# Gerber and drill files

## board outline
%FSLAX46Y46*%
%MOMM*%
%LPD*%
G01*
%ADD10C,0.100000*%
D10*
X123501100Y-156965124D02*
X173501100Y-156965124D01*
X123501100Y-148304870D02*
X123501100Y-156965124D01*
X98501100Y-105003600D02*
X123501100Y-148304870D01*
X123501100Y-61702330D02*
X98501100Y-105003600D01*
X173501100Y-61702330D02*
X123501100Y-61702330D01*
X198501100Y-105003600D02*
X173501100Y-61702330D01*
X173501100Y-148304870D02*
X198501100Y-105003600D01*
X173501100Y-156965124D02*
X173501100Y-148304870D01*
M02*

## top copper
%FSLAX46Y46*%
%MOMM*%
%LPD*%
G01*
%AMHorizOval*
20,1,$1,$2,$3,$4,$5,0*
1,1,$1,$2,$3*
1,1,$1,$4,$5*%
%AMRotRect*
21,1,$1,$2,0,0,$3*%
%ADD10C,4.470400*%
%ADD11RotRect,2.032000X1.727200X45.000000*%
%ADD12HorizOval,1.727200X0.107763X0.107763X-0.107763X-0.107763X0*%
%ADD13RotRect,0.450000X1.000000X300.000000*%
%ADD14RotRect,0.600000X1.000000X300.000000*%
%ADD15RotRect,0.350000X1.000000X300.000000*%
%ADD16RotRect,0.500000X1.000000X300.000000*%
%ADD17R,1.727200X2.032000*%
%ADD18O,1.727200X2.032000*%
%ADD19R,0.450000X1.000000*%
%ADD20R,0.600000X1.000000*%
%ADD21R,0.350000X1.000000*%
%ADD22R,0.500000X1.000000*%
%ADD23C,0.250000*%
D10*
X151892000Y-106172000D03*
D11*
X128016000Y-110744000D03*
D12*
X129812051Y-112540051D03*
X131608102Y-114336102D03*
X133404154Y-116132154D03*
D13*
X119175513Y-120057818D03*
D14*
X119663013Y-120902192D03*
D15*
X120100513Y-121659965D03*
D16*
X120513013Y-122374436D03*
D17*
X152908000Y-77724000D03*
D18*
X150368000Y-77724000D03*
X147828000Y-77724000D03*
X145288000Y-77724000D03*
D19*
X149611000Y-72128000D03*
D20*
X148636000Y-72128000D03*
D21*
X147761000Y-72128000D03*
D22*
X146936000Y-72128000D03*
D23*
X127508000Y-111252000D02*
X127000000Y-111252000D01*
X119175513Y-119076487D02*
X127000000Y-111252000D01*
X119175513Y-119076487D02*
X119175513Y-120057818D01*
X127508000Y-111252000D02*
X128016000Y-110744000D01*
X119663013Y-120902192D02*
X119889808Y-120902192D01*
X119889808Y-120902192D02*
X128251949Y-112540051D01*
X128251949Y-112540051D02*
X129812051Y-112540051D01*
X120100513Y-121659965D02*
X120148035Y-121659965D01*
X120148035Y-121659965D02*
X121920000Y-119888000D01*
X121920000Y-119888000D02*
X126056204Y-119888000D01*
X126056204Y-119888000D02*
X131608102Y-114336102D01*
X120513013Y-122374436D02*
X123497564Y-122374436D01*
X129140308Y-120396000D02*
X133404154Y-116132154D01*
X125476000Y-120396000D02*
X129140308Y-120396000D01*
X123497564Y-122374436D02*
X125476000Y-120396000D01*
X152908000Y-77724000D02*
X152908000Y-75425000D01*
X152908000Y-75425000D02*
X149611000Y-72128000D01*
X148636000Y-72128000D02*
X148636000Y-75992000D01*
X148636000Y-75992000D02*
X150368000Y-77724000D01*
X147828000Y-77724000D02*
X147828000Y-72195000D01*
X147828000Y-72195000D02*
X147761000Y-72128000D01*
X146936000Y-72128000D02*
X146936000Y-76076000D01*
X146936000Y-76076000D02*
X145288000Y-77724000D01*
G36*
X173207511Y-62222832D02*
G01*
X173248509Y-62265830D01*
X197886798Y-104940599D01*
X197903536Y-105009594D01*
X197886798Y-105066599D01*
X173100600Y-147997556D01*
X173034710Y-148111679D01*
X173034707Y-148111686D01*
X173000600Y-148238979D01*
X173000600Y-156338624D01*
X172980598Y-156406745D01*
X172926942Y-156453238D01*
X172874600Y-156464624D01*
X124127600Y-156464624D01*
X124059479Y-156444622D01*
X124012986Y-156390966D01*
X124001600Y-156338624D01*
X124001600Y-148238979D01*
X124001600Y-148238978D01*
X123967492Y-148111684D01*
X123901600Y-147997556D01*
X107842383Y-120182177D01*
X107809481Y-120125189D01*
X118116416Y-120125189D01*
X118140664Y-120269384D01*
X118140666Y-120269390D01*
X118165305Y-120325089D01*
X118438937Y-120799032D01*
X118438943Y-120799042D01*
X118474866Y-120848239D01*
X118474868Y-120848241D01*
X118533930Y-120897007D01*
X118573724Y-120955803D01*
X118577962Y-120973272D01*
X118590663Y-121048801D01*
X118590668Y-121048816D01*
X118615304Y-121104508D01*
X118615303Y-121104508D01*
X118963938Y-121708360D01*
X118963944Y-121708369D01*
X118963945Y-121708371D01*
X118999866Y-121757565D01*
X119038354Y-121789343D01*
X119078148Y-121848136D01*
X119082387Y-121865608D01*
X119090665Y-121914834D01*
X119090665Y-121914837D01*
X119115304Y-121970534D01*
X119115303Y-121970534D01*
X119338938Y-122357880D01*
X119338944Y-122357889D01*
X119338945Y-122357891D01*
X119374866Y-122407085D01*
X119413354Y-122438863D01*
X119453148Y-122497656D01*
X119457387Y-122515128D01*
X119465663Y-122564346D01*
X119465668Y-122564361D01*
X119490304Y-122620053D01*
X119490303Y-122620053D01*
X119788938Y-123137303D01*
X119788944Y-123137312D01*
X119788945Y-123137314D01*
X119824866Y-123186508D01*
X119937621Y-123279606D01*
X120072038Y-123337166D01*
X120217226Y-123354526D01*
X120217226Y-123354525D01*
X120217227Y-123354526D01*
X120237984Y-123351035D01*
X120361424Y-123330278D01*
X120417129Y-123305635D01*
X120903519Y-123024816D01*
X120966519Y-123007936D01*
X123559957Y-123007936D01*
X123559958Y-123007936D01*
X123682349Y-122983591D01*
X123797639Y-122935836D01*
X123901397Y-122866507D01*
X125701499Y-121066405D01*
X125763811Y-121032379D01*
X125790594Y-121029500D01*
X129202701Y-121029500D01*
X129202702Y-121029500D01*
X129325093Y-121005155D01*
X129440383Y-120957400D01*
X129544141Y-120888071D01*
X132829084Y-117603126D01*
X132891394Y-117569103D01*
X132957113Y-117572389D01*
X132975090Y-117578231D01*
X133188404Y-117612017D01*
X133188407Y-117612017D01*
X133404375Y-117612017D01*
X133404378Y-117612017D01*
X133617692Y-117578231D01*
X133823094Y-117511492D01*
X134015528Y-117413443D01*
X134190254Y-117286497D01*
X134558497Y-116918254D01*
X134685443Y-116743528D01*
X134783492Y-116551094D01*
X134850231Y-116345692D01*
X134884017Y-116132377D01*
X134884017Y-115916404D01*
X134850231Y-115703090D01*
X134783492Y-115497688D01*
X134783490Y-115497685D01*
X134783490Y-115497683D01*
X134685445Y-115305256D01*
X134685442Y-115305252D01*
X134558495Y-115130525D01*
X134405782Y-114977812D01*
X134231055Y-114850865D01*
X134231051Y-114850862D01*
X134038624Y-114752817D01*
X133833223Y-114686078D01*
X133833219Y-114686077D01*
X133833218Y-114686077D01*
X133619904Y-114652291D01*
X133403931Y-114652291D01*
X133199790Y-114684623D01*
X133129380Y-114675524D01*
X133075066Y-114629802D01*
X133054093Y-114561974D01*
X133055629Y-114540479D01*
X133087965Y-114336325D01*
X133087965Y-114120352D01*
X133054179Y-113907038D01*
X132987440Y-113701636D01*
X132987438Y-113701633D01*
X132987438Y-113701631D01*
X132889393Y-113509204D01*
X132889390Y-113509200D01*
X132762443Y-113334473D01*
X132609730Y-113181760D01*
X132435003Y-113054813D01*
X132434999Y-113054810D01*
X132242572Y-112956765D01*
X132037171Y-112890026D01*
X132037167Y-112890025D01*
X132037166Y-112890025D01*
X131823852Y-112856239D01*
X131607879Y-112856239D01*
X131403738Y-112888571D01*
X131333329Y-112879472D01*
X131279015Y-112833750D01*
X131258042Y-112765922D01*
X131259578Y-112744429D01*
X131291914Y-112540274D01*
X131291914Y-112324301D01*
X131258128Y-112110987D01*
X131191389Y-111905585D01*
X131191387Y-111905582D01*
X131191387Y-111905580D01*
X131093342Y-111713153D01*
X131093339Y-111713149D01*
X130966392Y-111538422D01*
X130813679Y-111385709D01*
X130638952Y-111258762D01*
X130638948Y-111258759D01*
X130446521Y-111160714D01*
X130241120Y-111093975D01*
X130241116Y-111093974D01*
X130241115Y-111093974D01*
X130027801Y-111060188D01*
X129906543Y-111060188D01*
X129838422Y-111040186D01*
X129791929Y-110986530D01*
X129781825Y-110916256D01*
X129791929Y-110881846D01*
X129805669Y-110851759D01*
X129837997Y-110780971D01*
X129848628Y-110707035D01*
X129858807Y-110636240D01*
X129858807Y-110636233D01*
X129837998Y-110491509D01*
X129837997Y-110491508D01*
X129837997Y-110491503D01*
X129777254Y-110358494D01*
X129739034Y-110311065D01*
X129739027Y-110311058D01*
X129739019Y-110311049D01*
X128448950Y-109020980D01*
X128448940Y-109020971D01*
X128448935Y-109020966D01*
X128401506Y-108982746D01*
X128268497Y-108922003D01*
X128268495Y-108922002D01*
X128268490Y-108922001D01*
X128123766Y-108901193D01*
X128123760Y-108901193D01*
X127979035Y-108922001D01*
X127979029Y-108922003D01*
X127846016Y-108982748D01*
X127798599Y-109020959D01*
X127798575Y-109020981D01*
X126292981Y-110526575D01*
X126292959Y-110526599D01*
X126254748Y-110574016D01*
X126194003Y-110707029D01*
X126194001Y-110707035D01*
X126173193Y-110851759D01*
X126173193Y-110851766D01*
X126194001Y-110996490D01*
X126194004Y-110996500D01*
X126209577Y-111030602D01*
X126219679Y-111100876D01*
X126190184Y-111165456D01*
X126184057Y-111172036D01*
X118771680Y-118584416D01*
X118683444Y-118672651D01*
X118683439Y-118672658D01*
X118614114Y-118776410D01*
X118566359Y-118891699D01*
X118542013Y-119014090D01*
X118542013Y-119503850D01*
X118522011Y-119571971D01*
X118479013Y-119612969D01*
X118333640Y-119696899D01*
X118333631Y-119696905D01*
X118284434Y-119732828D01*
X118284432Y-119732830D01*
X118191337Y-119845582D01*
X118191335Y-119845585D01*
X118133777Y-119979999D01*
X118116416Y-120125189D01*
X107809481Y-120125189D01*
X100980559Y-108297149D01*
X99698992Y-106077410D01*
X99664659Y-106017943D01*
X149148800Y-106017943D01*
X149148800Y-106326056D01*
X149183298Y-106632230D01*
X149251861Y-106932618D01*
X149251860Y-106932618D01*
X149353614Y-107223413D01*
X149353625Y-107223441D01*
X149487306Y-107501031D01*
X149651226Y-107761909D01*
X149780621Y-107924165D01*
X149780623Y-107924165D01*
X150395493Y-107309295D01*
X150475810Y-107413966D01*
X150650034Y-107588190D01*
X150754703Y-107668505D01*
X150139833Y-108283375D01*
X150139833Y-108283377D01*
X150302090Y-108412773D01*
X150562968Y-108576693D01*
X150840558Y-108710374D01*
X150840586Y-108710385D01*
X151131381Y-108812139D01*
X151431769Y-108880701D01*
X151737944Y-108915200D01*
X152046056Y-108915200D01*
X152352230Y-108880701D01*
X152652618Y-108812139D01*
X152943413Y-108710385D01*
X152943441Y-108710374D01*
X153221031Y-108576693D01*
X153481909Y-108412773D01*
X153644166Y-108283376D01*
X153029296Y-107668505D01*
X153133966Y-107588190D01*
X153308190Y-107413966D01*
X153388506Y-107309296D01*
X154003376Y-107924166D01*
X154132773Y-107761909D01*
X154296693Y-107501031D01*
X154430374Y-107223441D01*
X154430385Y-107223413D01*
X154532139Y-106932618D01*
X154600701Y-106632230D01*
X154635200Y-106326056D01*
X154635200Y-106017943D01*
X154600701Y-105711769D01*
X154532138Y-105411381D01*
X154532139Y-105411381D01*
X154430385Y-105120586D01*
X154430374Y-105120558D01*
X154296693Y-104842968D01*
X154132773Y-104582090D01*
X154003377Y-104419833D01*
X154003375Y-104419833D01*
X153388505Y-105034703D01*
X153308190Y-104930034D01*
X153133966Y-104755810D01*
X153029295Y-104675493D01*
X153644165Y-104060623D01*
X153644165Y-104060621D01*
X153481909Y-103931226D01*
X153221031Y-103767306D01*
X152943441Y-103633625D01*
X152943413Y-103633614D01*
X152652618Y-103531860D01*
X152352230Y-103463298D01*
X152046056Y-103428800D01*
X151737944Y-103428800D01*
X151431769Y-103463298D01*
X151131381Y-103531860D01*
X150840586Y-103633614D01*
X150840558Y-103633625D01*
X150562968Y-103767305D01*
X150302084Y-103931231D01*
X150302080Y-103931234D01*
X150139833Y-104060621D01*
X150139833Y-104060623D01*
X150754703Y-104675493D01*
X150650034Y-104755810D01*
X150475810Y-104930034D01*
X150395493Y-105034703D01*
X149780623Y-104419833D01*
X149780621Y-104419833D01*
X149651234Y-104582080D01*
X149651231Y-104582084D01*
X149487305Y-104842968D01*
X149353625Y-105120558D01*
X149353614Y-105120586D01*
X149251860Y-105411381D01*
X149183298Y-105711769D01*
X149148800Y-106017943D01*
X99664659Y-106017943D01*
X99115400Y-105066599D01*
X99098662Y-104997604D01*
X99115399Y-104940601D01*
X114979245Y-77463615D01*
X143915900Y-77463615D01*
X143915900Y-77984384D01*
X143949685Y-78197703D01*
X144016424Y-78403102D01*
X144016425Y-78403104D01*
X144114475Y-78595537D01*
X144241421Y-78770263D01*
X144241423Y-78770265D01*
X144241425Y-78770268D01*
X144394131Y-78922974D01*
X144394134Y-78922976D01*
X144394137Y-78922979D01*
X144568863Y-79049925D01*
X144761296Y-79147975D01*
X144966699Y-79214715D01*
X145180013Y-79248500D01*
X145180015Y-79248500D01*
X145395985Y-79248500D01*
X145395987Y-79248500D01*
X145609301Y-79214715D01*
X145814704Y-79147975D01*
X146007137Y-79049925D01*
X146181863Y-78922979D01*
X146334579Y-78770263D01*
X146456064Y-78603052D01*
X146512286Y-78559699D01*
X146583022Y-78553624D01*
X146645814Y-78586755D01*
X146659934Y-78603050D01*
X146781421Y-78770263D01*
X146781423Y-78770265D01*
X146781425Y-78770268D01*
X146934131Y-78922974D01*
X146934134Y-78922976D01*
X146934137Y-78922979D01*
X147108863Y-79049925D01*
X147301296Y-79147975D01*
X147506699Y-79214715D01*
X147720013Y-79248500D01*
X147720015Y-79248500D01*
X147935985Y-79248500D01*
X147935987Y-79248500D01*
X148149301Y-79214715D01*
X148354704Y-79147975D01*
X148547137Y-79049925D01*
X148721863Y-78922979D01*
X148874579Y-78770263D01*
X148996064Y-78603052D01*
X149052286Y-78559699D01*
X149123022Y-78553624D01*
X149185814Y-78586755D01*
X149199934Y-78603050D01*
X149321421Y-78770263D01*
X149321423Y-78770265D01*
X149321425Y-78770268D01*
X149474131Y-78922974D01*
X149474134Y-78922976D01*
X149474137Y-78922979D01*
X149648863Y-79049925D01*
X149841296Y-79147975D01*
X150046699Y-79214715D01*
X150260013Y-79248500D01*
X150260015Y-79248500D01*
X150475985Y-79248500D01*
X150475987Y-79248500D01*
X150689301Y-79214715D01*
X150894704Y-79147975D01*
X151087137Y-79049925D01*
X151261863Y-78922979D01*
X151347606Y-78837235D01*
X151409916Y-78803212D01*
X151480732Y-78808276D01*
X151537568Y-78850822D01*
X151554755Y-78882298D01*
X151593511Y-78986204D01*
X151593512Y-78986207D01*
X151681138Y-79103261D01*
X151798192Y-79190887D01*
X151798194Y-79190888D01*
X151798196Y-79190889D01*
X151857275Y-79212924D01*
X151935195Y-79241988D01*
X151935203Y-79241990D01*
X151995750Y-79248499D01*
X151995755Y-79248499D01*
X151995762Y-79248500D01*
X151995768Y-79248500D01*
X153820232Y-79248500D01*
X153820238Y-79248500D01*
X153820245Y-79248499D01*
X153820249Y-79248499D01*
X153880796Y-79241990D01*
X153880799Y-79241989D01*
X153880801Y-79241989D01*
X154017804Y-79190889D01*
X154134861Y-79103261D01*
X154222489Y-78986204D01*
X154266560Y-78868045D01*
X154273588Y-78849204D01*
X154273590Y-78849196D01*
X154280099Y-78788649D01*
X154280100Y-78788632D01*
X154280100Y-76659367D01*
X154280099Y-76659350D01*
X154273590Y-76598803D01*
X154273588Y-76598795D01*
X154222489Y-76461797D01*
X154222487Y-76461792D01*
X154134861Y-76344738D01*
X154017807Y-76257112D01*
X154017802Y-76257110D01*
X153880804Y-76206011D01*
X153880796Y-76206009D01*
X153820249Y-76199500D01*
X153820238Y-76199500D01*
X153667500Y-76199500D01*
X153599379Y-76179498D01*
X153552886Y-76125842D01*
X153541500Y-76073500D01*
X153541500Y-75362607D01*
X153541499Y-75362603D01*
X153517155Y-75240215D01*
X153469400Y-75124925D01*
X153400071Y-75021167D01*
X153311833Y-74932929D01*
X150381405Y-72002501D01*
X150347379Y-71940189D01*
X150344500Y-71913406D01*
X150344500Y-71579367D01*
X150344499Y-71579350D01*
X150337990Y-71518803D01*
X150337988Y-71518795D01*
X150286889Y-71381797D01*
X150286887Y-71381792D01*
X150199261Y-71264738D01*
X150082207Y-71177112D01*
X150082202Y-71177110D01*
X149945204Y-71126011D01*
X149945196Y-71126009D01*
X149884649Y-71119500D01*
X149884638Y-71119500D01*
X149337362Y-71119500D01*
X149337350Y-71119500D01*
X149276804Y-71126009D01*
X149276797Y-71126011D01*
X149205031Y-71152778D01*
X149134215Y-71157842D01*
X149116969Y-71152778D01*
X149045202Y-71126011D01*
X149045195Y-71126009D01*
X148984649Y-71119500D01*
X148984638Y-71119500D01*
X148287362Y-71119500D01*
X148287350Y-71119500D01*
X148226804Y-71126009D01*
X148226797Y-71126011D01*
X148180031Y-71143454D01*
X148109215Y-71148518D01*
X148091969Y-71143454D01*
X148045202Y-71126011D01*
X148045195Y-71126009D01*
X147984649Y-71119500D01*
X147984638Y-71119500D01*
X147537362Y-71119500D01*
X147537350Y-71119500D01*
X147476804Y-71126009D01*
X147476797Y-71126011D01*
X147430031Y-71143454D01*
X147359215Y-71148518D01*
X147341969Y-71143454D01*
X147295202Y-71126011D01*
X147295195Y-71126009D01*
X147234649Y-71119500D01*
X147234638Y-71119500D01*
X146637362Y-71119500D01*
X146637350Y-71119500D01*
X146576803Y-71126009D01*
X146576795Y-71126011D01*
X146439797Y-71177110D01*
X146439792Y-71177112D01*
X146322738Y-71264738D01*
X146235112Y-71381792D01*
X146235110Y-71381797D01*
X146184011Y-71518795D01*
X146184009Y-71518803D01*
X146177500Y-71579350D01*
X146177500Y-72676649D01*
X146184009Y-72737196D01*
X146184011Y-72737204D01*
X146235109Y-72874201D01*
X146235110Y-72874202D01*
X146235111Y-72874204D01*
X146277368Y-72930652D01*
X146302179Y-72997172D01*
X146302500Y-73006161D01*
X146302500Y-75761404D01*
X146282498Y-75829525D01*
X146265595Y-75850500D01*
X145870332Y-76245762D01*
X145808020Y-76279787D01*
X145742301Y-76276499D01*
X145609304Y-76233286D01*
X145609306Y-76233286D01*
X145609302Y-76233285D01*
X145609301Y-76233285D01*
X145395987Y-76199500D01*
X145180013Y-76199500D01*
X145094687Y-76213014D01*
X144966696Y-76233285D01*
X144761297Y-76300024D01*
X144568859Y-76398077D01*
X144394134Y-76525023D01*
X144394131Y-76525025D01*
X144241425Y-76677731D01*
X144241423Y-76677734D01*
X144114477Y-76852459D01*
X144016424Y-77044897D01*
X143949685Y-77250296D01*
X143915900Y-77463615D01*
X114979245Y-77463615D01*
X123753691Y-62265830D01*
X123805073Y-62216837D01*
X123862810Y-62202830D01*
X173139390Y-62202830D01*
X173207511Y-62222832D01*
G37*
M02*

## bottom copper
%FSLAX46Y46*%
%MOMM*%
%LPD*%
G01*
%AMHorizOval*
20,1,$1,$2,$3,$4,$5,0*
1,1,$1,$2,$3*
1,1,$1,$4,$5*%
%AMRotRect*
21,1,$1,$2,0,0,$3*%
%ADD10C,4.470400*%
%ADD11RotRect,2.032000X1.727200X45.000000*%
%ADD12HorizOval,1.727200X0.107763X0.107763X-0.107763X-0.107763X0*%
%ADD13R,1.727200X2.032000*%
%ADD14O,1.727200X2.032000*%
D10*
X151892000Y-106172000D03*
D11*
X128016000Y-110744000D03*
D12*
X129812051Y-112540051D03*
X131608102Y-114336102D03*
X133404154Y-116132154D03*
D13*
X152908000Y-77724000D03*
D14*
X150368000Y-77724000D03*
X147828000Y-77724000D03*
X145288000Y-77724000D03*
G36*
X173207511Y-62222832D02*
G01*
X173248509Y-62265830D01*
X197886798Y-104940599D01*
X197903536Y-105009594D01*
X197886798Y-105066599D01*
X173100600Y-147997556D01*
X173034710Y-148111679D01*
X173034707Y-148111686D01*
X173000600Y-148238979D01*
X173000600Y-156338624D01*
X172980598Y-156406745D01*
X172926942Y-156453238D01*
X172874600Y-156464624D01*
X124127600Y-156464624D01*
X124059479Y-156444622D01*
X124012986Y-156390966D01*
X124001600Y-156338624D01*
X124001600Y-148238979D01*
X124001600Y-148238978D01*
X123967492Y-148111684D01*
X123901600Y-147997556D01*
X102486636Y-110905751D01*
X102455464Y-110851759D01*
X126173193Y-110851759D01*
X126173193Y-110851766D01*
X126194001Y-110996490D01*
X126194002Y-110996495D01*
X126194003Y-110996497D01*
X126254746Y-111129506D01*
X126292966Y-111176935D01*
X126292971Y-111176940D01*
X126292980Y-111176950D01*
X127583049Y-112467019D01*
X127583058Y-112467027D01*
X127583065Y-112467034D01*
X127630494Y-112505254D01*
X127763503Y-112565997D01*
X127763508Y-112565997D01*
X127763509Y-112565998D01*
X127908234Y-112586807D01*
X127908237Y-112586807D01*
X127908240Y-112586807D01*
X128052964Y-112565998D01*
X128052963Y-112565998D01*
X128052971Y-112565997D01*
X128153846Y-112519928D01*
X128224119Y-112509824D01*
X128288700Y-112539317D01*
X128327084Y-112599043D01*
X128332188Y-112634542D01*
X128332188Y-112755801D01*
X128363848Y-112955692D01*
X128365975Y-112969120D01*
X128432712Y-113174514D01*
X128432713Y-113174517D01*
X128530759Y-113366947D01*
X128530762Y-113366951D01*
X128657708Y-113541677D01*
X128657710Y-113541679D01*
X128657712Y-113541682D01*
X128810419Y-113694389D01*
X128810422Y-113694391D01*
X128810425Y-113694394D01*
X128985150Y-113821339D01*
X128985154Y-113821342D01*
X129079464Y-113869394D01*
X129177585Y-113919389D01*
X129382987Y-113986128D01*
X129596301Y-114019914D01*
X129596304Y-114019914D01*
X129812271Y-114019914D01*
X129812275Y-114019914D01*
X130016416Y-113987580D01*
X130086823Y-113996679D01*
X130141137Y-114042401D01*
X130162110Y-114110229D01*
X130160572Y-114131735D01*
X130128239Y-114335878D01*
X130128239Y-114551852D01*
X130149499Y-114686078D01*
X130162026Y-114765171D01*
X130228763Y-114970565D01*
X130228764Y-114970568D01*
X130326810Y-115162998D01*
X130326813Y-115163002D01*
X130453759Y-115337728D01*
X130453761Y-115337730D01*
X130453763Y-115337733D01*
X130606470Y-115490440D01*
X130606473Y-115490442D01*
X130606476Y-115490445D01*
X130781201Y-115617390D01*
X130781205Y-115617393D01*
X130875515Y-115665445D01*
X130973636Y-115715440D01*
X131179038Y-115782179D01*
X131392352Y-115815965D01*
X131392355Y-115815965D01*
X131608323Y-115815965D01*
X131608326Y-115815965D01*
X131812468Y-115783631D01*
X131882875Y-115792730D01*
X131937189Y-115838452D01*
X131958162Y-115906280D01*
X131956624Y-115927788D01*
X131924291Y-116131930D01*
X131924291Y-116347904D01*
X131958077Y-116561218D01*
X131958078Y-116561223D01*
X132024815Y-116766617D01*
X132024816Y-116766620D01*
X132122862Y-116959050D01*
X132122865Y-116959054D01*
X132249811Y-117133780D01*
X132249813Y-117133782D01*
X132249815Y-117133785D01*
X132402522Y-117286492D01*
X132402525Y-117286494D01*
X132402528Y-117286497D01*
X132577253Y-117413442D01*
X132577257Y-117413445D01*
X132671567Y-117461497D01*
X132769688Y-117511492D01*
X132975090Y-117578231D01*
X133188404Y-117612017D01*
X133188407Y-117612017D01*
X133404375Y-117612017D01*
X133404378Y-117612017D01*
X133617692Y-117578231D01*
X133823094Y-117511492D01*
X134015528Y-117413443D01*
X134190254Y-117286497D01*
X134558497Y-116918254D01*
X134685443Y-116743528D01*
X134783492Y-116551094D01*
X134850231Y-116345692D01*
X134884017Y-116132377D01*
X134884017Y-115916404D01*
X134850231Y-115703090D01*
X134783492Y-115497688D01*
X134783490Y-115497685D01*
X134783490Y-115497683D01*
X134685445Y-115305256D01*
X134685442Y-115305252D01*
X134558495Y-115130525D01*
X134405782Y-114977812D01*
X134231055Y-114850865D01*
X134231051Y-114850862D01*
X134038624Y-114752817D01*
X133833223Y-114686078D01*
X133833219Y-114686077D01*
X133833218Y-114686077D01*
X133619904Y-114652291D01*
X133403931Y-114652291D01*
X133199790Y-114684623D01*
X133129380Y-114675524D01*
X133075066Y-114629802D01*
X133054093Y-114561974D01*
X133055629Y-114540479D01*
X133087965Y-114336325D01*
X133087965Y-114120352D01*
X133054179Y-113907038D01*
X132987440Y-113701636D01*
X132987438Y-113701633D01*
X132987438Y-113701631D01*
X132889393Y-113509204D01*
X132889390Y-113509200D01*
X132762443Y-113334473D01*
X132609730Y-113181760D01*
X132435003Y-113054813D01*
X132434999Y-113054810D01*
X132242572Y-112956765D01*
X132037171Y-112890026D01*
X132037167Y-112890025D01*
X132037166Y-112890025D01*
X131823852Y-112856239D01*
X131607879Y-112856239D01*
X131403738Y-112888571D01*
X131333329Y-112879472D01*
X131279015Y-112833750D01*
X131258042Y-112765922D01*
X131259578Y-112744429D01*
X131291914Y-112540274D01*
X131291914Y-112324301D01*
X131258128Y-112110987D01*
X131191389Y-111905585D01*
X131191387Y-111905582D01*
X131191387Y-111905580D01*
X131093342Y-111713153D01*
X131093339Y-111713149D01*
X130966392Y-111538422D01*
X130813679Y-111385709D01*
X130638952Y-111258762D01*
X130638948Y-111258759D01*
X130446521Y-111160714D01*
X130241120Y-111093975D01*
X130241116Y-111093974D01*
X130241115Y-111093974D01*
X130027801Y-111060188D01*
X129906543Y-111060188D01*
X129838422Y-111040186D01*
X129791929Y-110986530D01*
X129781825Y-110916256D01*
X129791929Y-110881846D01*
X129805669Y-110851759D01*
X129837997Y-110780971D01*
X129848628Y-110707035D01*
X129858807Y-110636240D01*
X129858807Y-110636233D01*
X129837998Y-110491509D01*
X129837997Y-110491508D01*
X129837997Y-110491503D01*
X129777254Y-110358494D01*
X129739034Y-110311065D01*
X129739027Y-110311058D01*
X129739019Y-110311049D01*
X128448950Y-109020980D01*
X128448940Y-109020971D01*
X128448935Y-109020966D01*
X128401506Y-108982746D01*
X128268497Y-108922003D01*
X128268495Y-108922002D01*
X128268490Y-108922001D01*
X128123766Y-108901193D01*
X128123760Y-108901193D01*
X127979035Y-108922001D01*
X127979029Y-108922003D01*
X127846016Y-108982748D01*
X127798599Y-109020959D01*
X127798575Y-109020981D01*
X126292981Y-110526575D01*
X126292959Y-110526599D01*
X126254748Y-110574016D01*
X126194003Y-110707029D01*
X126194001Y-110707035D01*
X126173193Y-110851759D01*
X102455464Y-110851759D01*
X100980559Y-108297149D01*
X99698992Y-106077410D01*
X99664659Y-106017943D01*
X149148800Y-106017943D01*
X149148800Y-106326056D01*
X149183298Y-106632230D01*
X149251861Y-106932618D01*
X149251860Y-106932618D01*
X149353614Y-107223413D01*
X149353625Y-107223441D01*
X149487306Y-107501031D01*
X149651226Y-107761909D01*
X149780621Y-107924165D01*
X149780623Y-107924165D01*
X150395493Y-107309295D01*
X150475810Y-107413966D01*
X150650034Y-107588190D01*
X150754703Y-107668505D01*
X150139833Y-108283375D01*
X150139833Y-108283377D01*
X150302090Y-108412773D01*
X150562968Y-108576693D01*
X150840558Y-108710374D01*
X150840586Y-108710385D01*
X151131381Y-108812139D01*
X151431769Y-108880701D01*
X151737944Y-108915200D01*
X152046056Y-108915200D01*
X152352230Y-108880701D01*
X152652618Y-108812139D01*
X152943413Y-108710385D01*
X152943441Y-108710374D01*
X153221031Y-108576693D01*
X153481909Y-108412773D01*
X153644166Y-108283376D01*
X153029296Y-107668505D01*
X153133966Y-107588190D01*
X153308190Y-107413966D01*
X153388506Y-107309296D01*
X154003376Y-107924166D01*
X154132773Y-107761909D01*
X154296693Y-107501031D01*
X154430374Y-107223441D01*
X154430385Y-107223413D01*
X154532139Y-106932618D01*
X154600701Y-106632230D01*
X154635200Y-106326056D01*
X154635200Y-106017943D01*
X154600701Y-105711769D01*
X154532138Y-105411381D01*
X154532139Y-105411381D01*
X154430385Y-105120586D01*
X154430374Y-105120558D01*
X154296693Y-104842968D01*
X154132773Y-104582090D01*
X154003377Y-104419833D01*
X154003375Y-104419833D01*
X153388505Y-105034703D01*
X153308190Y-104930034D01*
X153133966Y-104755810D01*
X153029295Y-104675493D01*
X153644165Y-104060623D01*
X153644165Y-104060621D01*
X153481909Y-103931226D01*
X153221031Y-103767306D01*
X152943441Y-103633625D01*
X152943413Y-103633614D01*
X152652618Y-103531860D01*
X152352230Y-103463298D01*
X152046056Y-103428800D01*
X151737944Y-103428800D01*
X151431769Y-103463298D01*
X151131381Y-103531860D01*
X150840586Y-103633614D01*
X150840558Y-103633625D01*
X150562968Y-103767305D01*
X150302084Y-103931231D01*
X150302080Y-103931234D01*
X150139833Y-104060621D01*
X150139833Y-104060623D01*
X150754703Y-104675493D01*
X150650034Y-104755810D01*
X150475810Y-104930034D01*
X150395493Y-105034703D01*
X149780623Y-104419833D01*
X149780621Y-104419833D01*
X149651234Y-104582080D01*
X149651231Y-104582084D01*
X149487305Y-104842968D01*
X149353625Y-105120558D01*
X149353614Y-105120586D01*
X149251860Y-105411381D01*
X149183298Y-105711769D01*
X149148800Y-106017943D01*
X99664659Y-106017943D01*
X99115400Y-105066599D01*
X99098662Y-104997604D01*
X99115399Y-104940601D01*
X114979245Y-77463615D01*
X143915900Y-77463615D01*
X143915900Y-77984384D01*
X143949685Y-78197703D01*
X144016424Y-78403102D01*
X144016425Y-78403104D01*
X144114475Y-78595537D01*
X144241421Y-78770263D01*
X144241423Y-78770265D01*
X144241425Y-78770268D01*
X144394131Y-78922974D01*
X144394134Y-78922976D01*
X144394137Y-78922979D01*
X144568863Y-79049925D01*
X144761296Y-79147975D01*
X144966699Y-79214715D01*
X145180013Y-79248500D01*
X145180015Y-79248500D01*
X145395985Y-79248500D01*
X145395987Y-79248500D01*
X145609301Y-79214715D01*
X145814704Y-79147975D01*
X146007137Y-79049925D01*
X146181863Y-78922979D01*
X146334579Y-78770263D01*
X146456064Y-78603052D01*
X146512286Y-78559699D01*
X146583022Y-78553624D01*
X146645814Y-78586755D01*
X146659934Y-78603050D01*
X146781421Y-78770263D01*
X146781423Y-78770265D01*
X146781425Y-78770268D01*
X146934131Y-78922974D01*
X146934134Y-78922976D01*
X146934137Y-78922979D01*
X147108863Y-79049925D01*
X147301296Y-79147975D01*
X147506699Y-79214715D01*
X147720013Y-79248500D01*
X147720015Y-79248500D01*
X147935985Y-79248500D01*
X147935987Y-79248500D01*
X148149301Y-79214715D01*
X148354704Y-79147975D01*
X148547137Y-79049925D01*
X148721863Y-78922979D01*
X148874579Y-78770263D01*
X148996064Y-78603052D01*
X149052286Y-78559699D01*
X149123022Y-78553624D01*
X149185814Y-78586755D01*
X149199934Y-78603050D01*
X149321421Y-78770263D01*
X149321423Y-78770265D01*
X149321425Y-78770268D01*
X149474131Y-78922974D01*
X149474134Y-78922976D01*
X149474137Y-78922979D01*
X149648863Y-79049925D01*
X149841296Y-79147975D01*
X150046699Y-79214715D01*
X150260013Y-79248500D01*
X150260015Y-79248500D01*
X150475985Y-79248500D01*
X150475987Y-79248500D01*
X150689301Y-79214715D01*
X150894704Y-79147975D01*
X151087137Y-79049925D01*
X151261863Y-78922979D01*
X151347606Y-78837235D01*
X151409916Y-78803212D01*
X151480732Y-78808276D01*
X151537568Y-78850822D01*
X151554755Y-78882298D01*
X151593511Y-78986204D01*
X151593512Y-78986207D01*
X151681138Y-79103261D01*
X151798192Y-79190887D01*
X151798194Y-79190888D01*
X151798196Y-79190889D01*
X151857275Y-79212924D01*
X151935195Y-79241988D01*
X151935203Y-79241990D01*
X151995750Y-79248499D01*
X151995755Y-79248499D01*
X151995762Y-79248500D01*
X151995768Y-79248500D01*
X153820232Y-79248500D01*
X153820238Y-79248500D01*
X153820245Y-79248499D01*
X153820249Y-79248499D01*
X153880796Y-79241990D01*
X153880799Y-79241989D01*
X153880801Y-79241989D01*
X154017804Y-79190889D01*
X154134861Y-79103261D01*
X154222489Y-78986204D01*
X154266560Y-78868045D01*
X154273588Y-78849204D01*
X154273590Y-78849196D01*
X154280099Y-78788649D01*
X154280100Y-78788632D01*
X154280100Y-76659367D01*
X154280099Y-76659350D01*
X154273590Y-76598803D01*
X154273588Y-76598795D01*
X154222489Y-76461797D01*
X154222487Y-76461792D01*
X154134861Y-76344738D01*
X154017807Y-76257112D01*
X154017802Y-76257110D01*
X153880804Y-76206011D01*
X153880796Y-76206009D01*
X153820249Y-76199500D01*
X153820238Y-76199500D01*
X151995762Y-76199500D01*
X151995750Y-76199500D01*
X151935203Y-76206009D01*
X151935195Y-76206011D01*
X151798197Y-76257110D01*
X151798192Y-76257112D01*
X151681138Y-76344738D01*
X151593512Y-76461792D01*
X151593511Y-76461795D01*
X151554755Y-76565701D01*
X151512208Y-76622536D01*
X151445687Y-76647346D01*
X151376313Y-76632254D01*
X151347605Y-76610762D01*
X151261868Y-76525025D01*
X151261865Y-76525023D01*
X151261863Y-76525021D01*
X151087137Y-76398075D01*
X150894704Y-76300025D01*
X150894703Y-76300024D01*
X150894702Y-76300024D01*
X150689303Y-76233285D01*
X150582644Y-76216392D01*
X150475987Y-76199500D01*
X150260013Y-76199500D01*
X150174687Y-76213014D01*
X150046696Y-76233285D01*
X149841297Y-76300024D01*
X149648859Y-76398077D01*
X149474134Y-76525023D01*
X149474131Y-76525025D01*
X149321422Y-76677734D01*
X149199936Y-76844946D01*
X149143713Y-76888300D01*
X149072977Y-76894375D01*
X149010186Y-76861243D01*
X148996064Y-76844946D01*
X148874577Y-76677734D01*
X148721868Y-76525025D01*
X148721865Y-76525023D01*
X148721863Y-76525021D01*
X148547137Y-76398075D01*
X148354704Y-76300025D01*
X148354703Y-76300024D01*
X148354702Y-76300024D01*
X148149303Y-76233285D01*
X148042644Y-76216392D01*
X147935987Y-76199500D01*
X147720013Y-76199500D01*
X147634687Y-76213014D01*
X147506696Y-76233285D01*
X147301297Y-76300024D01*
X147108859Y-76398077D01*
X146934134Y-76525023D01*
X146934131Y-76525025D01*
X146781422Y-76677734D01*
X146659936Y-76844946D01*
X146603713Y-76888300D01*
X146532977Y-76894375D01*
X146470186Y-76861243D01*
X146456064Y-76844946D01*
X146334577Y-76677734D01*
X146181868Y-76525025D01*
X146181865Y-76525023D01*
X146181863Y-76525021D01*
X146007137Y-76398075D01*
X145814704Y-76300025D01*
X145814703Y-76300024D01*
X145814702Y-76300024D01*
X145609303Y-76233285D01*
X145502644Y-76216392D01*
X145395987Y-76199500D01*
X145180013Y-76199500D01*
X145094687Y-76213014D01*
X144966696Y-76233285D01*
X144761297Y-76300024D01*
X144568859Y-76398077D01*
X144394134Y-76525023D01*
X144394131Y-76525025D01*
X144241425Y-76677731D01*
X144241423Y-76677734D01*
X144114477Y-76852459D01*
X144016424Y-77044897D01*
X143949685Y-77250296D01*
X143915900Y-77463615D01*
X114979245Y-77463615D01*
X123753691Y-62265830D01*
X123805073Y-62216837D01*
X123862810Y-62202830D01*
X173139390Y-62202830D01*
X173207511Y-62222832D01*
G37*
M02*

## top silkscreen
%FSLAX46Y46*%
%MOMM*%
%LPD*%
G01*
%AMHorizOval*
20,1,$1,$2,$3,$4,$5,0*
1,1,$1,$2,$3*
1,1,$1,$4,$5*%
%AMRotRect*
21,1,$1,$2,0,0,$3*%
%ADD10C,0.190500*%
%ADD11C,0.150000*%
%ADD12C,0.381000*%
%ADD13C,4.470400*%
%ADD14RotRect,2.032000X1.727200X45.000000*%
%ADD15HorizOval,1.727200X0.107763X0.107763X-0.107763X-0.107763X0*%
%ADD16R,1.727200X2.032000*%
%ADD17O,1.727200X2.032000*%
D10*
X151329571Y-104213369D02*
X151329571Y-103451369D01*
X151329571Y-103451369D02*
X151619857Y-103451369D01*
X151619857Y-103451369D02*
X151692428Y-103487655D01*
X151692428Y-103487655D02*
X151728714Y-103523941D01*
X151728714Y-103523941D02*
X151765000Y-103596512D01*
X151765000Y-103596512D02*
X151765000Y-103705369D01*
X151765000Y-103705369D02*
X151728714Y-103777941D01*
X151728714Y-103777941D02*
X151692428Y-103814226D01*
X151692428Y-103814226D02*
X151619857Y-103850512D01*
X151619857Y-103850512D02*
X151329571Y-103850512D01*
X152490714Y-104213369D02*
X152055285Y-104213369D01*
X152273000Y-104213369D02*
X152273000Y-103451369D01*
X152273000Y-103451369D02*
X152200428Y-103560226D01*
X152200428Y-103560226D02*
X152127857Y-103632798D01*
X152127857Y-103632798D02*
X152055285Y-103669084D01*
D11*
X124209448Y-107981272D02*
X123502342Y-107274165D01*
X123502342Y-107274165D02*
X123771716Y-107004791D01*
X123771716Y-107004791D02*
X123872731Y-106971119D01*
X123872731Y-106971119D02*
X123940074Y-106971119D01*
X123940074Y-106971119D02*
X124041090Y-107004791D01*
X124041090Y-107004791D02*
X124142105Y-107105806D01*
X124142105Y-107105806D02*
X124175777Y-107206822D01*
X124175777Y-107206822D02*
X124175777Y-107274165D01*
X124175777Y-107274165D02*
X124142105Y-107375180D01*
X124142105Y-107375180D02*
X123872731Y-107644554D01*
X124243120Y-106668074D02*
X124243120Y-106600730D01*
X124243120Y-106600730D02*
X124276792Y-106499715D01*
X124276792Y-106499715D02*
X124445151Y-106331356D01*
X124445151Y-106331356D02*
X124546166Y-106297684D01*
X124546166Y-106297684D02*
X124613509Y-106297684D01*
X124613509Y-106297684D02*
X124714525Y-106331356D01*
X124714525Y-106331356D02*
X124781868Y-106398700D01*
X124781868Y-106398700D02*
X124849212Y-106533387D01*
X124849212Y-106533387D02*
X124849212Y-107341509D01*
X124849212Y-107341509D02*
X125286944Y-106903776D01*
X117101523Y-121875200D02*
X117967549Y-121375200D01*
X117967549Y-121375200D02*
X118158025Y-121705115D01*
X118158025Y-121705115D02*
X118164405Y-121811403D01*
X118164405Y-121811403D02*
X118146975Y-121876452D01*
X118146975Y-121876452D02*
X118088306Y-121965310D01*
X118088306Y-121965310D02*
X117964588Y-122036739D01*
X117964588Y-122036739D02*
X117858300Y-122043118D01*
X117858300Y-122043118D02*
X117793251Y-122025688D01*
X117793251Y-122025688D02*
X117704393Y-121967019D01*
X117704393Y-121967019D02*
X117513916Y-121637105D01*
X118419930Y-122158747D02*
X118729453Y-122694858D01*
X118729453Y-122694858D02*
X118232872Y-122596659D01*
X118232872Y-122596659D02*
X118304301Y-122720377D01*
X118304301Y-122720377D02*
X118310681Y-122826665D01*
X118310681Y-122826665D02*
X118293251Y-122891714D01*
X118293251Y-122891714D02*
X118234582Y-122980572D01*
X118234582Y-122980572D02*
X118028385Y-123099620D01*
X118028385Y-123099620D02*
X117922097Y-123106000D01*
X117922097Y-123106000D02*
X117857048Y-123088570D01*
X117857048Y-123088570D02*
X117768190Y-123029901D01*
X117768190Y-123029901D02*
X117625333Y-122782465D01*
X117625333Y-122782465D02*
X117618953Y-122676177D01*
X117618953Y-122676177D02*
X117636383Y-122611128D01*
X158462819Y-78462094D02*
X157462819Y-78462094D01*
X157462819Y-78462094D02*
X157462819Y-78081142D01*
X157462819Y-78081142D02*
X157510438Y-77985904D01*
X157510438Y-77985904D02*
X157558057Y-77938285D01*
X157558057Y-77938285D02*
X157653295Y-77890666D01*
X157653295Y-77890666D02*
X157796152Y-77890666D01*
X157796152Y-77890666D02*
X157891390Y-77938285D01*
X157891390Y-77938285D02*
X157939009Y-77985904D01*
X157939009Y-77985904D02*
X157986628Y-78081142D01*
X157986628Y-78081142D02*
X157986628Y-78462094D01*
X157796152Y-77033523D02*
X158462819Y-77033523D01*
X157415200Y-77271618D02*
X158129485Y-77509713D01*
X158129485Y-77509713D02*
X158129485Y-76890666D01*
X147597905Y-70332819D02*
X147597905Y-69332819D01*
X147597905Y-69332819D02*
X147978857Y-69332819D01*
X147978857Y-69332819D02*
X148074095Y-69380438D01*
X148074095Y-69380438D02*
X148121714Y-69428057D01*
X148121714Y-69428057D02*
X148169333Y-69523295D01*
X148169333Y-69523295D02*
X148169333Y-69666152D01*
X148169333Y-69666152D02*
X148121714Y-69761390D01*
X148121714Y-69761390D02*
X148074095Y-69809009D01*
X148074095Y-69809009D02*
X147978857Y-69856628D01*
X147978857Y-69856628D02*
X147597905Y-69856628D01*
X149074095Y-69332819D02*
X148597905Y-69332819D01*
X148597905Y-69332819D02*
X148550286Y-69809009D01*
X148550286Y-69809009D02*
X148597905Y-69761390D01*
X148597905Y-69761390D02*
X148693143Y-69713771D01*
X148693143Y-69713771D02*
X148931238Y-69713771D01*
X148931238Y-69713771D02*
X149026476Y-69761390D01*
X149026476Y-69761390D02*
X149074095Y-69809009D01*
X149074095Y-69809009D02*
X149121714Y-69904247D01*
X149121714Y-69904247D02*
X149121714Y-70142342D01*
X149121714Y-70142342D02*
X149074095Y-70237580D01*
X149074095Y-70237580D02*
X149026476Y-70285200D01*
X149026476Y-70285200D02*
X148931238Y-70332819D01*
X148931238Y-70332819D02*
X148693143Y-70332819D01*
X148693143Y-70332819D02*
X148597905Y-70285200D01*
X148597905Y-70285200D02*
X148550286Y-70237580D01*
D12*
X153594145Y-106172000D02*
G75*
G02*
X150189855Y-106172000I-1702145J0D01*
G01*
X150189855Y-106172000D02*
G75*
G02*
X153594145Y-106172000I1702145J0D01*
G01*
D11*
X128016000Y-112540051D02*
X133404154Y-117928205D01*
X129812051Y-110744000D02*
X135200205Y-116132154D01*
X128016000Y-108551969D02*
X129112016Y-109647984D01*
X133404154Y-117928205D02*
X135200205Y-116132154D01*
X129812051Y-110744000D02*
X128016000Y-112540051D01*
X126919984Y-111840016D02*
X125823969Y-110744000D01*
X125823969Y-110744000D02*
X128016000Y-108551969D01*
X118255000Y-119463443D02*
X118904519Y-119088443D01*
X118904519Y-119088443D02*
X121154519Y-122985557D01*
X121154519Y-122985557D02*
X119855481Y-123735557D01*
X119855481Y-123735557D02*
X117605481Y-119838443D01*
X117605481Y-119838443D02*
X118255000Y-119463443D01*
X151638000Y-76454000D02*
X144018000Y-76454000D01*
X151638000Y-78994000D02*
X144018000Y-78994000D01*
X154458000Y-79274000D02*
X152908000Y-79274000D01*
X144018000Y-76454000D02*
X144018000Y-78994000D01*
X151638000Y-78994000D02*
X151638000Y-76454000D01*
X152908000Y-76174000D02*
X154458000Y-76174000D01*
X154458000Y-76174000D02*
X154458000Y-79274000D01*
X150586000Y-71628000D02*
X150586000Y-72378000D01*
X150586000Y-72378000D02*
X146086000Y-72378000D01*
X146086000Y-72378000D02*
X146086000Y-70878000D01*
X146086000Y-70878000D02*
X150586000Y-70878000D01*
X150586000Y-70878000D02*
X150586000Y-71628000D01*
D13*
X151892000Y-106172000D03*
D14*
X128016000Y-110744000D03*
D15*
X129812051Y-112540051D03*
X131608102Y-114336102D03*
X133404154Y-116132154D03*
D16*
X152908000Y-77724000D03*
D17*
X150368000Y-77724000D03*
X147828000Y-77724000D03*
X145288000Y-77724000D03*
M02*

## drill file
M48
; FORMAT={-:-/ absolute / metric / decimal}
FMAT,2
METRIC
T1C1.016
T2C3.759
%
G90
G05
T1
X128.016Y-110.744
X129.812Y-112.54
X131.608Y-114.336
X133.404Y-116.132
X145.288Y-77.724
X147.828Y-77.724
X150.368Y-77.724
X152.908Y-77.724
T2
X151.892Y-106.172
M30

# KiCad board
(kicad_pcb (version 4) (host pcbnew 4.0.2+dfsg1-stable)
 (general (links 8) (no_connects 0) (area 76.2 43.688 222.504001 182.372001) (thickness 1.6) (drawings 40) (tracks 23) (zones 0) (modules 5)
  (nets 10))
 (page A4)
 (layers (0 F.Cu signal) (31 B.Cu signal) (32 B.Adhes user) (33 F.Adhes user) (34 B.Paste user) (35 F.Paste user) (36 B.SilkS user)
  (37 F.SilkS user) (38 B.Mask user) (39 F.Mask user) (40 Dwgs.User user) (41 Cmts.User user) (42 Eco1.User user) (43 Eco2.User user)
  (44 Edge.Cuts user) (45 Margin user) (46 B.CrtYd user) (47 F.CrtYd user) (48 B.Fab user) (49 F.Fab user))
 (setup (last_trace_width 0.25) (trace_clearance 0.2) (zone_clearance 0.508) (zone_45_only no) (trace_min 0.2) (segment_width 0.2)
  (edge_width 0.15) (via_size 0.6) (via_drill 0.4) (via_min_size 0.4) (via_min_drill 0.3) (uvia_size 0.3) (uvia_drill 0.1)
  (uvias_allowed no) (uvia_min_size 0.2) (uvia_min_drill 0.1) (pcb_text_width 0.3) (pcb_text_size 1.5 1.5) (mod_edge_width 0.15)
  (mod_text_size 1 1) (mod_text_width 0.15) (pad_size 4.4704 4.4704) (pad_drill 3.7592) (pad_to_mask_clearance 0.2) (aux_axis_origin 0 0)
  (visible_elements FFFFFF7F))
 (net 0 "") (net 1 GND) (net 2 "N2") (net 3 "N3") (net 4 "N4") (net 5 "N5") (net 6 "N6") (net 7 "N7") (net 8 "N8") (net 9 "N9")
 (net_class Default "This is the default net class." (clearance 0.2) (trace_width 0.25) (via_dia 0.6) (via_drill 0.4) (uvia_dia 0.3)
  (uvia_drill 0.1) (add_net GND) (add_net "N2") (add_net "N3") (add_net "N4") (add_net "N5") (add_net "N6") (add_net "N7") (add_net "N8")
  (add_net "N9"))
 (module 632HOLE (layer F.Cu) (at 151.892 106.172)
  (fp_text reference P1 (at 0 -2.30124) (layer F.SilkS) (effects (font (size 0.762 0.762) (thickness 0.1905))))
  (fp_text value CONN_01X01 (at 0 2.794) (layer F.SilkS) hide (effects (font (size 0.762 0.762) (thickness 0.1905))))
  (fp_circle (center 0 0) (end 1.69926 -0.09906) (layer F.SilkS) (width 0.381))
  (pad 1 thru_hole circle (at 0 0) (size 4.4704 4.4704) (drill 3.7592) (layers *.Cu *.Mask F.SilkS) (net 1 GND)))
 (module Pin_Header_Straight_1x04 (layer F.Cu) (at 128.016 110.744 45)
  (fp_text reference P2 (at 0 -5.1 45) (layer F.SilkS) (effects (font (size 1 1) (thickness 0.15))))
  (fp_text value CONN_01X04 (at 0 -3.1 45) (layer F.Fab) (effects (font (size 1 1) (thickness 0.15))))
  (fp_line (start -1.27 1.27) (end -1.27 8.89) (layer F.SilkS) (width 0.15))
  (fp_line (start 1.27 1.27) (end 1.27 8.89) (layer F.SilkS) (width 0.15))
  (fp_line (start 1.55 -1.55) (end 1.55 0) (layer F.SilkS) (width 0.15))
  (fp_line (start -1.27 8.89) (end 1.27 8.89) (layer F.SilkS) (width 0.15))
  (fp_line (start 1.27 1.27) (end -1.27 1.27) (layer F.SilkS) (width 0.15))
  (fp_line (start -1.55 0) (end -1.55 -1.55) (layer F.SilkS) (width 0.15))
  (fp_line (start -1.55 -1.55) (end 1.55 -1.55) (layer F.SilkS) (width 0.15))
  (pad 1 thru_hole rect (at 0 0 45) (size 2.032 1.7272) (drill 1.016) (layers *.Cu *.Mask F.SilkS) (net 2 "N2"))
  (pad 2 thru_hole oval (at 0 2.54 45) (size 2.032 1.7272) (drill 1.016) (layers *.Cu *.Mask F.SilkS) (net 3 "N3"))
  (pad 3 thru_hole oval (at 0 5.08 45) (size 2.032 1.7272) (drill 1.016) (layers *.Cu *.Mask F.SilkS) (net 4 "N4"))
  (pad 4 thru_hole oval (at 0 7.62 45) (size 2.032 1.7272) (drill 1.016) (layers *.Cu *.Mask F.SilkS) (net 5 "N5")))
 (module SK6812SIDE (layer F.Cu) (at 119.38 121.412 300)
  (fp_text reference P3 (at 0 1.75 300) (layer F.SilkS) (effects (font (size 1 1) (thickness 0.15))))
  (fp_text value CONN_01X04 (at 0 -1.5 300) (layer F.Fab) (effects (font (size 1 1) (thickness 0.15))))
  (fp_line (start -2.25 0) (end -2.25 -0.75) (layer F.SilkS) (width 0.15))
  (fp_line (start -2.25 -0.75) (end 2.25 -0.75) (layer F.SilkS) (width 0.15))
  (fp_line (start 2.25 -0.75) (end 2.25 0.75) (layer F.SilkS) (width 0.15))
  (fp_line (start 2.25 0.75) (end -2.25 0.75) (layer F.SilkS) (width 0.15))
  (fp_line (start -2.25 0.75) (end -2.25 0) (layer F.SilkS) (width 0.15))
  (pad 1 smd rect (at -1.275 -0.5 300) (size 0.45 1) (layers F.Cu F.Paste F.Mask) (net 2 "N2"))
  (pad 2 smd rect (at -0.3 -0.5 300) (size 0.6 1) (layers F.Cu F.Paste F.Mask) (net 3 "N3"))
  (pad 3 smd rect (at 0.575 -0.5 300) (size 0.35 1) (layers F.Cu F.Paste F.Mask) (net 4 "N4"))
  (pad 4 smd rect (at 1.4 -0.5 300) (size 0.5 1) (layers F.Cu F.Paste F.Mask) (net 5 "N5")))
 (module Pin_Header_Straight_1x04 (layer F.Cu) (at 152.908 77.724 270)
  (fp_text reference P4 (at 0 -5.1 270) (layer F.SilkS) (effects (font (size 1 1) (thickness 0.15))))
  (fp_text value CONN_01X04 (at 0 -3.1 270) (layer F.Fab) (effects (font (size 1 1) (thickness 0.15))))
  (fp_line (start -1.27 1.27) (end -1.27 8.89) (layer F.SilkS) (width 0.15))
  (fp_line (start 1.27 1.27) (end 1.27 8.89) (layer F.SilkS) (width 0.15))
  (fp_line (start 1.55 -1.55) (end 1.55 0) (layer F.SilkS) (width 0.15))
  (fp_line (start -1.27 8.89) (end 1.27 8.89) (layer F.SilkS) (width 0.15))
  (fp_line (start 1.27 1.27) (end -1.27 1.27) (layer F.SilkS) (width 0.15))
  (fp_line (start -1.55 0) (end -1.55 -1.55) (layer F.SilkS) (width 0.15))
  (fp_line (start -1.55 -1.55) (end 1.55 -1.55) (layer F.SilkS) (width 0.15))
  (pad 1 thru_hole rect (at 0 0 270) (size 2.032 1.7272) (drill 1.016) (layers *.Cu *.Mask F.SilkS) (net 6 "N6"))
  (pad 2 thru_hole oval (at 0 2.54 270) (size 2.032 1.7272) (drill 1.016) (layers *.Cu *.Mask F.SilkS) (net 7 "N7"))
  (pad 3 thru_hole oval (at 0 5.08 270) (size 2.032 1.7272) (drill 1.016) (layers *.Cu *.Mask F.SilkS) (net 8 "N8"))
  (pad 4 thru_hole oval (at 0 7.62 270) (size 2.032 1.7272) (drill 1.016) (layers *.Cu *.Mask F.SilkS) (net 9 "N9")))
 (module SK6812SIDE (layer F.Cu) (at 148.336 71.628 180)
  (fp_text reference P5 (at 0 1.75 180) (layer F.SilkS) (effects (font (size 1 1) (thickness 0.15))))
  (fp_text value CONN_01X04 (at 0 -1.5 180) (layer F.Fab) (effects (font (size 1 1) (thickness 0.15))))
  (fp_line (start -2.25 0) (end -2.25 -0.75) (layer F.SilkS) (width 0.15))
  (fp_line (start -2.25 -0.75) (end 2.25 -0.75) (layer F.SilkS) (width 0.15))
  (fp_line (start 2.25 -0.75) (end 2.25 0.75) (layer F.SilkS) (width 0.15))
  (fp_line (start 2.25 0.75) (end -2.25 0.75) (layer F.SilkS) (width 0.15))
  (fp_line (start -2.25 0.75) (end -2.25 0) (layer F.SilkS) (width 0.15))
  (pad 1 smd rect (at -1.275 -0.5 180) (size 0.45 1) (layers F.Cu F.Paste F.Mask) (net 6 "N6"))
  (pad 2 smd rect (at -0.3 -0.5 180) (size 0.6 1) (layers F.Cu F.Paste F.Mask) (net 7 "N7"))
  (pad 3 smd rect (at 0.575 -0.5 180) (size 0.35 1) (layers F.Cu F.Paste F.Mask) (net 8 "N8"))
  (pad 4 smd rect (at 1.4 -0.5 180) (size 0.5 1) (layers F.Cu F.Paste F.Mask) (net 9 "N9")))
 (gr_line (start 123.5011 156.965124) (end 173.5011 156.965124) (layer Edge.Cuts) (width 0.1))
 (gr_line (start 123.5011 148.30487) (end 123.5011 156.965124) (layer Edge.Cuts) (width 0.1))
 (gr_line (start 98.5011 105.0036) (end 123.5011 148.30487) (layer Edge.Cuts) (width 0.1))
 (gr_line (start 123.5011 61.70233) (end 98.5011 105.0036) (layer Edge.Cuts) (width 0.1))
 (gr_line (start 173.5011 61.70233) (end 123.5011 61.70233) (layer Edge.Cuts) (width 0.1))
 (gr_line (start 198.5011 105.0036) (end 173.5011 61.70233) (layer Edge.Cuts) (width 0.1))
 (gr_line (start 173.5011 148.30487) (end 198.5011 105.0036) (layer Edge.Cuts) (width 0.1))
 (gr_line (start 173.5011 156.965124) (end 173.5011 148.30487) (layer Edge.Cuts) (width 0.1))
 (segment (start 127.508 111.252) (end 127 111.252) (width 0.25) (layer F.Cu) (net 2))
 (segment (start 119.175513 119.076487) (end 127 111.252) (width 0.25) (layer F.Cu) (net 2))
 (segment (start 119.175513 119.076487) (end 119.175513 120.057818) (width 0.25) (layer F.Cu) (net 2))
 (segment (start 127.508 111.252) (end 128.016 110.744) (width 0.25) (layer F.Cu) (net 2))
 (segment (start 119.663013 120.902192) (end 119.889808 120.902192) (width 0.25) (layer F.Cu) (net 3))
 (segment (start 119.889808 120.902192) (end 128.251949 112.540051) (width 0.25) (layer F.Cu) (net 3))
 (segment (start 128.251949 112.540051) (end 129.812051 112.540051) (width 0.25) (layer F.Cu) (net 3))
 (segment (start 120.100513 121.659965) (end 120.148035 121.659965) (width 0.25) (layer F.Cu) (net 4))
 (segment (start 120.148035 121.659965) (end 121.92 119.888) (width 0.25) (layer F.Cu) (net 4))
 (segment (start 121.92 119.888) (end 126.056204 119.888) (width 0.25) (layer F.Cu) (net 4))
 (segment (start 126.056204 119.888) (end 131.608102 114.336102) (width 0.25) (layer F.Cu) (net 4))
 (segment (start 120.513013 122.374436) (end 123.497564 122.374436) (width 0.25) (layer F.Cu) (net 5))
 (segment (start 129.140308 120.396) (end 133.404154 116.132154) (width 0.25) (layer F.Cu) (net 5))
 (segment (start 125.476 120.396) (end 129.140308 120.396) (width 0.25) (layer F.Cu) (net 5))
 (segment (start 123.497564 122.374436) (end 125.476 120.396) (width 0.25) (layer F.Cu) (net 5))
 (segment (start 152.908 77.724) (end 152.908 75.425) (width 0.25) (layer F.Cu) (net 6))
 (segment (start 152.908 75.425) (end 149.611 72.128) (width 0.25) (layer F.Cu) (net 6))
 (segment (start 148.636 72.128) (end 148.636 75.992) (width 0.25) (layer F.Cu) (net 7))
 (segment (start 148.636 75.992) (end 150.368 77.724) (width 0.25) (layer F.Cu) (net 7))
 (segment (start 147.828 77.724) (end 147.828 72.195) (width 0.25) (layer F.Cu) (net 8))
 (segment (start 147.828 72.195) (end 147.761 72.128) (width 0.25) (layer F.Cu) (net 8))
 (segment (start 146.936 72.128) (end 146.936 76.076) (width 0.25) (layer F.Cu) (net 9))
 (segment (start 146.936 76.076) (end 145.288 77.724) (width 0.25) (layer F.Cu) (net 9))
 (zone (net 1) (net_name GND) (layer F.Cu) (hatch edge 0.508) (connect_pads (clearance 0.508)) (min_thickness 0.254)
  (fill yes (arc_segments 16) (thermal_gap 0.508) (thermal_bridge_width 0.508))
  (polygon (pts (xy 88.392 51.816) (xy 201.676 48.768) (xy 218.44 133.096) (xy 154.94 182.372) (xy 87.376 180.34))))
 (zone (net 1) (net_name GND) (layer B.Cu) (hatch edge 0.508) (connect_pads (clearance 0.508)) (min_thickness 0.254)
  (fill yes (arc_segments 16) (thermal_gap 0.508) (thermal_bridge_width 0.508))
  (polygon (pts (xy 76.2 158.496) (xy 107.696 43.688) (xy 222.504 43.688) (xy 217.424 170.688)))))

